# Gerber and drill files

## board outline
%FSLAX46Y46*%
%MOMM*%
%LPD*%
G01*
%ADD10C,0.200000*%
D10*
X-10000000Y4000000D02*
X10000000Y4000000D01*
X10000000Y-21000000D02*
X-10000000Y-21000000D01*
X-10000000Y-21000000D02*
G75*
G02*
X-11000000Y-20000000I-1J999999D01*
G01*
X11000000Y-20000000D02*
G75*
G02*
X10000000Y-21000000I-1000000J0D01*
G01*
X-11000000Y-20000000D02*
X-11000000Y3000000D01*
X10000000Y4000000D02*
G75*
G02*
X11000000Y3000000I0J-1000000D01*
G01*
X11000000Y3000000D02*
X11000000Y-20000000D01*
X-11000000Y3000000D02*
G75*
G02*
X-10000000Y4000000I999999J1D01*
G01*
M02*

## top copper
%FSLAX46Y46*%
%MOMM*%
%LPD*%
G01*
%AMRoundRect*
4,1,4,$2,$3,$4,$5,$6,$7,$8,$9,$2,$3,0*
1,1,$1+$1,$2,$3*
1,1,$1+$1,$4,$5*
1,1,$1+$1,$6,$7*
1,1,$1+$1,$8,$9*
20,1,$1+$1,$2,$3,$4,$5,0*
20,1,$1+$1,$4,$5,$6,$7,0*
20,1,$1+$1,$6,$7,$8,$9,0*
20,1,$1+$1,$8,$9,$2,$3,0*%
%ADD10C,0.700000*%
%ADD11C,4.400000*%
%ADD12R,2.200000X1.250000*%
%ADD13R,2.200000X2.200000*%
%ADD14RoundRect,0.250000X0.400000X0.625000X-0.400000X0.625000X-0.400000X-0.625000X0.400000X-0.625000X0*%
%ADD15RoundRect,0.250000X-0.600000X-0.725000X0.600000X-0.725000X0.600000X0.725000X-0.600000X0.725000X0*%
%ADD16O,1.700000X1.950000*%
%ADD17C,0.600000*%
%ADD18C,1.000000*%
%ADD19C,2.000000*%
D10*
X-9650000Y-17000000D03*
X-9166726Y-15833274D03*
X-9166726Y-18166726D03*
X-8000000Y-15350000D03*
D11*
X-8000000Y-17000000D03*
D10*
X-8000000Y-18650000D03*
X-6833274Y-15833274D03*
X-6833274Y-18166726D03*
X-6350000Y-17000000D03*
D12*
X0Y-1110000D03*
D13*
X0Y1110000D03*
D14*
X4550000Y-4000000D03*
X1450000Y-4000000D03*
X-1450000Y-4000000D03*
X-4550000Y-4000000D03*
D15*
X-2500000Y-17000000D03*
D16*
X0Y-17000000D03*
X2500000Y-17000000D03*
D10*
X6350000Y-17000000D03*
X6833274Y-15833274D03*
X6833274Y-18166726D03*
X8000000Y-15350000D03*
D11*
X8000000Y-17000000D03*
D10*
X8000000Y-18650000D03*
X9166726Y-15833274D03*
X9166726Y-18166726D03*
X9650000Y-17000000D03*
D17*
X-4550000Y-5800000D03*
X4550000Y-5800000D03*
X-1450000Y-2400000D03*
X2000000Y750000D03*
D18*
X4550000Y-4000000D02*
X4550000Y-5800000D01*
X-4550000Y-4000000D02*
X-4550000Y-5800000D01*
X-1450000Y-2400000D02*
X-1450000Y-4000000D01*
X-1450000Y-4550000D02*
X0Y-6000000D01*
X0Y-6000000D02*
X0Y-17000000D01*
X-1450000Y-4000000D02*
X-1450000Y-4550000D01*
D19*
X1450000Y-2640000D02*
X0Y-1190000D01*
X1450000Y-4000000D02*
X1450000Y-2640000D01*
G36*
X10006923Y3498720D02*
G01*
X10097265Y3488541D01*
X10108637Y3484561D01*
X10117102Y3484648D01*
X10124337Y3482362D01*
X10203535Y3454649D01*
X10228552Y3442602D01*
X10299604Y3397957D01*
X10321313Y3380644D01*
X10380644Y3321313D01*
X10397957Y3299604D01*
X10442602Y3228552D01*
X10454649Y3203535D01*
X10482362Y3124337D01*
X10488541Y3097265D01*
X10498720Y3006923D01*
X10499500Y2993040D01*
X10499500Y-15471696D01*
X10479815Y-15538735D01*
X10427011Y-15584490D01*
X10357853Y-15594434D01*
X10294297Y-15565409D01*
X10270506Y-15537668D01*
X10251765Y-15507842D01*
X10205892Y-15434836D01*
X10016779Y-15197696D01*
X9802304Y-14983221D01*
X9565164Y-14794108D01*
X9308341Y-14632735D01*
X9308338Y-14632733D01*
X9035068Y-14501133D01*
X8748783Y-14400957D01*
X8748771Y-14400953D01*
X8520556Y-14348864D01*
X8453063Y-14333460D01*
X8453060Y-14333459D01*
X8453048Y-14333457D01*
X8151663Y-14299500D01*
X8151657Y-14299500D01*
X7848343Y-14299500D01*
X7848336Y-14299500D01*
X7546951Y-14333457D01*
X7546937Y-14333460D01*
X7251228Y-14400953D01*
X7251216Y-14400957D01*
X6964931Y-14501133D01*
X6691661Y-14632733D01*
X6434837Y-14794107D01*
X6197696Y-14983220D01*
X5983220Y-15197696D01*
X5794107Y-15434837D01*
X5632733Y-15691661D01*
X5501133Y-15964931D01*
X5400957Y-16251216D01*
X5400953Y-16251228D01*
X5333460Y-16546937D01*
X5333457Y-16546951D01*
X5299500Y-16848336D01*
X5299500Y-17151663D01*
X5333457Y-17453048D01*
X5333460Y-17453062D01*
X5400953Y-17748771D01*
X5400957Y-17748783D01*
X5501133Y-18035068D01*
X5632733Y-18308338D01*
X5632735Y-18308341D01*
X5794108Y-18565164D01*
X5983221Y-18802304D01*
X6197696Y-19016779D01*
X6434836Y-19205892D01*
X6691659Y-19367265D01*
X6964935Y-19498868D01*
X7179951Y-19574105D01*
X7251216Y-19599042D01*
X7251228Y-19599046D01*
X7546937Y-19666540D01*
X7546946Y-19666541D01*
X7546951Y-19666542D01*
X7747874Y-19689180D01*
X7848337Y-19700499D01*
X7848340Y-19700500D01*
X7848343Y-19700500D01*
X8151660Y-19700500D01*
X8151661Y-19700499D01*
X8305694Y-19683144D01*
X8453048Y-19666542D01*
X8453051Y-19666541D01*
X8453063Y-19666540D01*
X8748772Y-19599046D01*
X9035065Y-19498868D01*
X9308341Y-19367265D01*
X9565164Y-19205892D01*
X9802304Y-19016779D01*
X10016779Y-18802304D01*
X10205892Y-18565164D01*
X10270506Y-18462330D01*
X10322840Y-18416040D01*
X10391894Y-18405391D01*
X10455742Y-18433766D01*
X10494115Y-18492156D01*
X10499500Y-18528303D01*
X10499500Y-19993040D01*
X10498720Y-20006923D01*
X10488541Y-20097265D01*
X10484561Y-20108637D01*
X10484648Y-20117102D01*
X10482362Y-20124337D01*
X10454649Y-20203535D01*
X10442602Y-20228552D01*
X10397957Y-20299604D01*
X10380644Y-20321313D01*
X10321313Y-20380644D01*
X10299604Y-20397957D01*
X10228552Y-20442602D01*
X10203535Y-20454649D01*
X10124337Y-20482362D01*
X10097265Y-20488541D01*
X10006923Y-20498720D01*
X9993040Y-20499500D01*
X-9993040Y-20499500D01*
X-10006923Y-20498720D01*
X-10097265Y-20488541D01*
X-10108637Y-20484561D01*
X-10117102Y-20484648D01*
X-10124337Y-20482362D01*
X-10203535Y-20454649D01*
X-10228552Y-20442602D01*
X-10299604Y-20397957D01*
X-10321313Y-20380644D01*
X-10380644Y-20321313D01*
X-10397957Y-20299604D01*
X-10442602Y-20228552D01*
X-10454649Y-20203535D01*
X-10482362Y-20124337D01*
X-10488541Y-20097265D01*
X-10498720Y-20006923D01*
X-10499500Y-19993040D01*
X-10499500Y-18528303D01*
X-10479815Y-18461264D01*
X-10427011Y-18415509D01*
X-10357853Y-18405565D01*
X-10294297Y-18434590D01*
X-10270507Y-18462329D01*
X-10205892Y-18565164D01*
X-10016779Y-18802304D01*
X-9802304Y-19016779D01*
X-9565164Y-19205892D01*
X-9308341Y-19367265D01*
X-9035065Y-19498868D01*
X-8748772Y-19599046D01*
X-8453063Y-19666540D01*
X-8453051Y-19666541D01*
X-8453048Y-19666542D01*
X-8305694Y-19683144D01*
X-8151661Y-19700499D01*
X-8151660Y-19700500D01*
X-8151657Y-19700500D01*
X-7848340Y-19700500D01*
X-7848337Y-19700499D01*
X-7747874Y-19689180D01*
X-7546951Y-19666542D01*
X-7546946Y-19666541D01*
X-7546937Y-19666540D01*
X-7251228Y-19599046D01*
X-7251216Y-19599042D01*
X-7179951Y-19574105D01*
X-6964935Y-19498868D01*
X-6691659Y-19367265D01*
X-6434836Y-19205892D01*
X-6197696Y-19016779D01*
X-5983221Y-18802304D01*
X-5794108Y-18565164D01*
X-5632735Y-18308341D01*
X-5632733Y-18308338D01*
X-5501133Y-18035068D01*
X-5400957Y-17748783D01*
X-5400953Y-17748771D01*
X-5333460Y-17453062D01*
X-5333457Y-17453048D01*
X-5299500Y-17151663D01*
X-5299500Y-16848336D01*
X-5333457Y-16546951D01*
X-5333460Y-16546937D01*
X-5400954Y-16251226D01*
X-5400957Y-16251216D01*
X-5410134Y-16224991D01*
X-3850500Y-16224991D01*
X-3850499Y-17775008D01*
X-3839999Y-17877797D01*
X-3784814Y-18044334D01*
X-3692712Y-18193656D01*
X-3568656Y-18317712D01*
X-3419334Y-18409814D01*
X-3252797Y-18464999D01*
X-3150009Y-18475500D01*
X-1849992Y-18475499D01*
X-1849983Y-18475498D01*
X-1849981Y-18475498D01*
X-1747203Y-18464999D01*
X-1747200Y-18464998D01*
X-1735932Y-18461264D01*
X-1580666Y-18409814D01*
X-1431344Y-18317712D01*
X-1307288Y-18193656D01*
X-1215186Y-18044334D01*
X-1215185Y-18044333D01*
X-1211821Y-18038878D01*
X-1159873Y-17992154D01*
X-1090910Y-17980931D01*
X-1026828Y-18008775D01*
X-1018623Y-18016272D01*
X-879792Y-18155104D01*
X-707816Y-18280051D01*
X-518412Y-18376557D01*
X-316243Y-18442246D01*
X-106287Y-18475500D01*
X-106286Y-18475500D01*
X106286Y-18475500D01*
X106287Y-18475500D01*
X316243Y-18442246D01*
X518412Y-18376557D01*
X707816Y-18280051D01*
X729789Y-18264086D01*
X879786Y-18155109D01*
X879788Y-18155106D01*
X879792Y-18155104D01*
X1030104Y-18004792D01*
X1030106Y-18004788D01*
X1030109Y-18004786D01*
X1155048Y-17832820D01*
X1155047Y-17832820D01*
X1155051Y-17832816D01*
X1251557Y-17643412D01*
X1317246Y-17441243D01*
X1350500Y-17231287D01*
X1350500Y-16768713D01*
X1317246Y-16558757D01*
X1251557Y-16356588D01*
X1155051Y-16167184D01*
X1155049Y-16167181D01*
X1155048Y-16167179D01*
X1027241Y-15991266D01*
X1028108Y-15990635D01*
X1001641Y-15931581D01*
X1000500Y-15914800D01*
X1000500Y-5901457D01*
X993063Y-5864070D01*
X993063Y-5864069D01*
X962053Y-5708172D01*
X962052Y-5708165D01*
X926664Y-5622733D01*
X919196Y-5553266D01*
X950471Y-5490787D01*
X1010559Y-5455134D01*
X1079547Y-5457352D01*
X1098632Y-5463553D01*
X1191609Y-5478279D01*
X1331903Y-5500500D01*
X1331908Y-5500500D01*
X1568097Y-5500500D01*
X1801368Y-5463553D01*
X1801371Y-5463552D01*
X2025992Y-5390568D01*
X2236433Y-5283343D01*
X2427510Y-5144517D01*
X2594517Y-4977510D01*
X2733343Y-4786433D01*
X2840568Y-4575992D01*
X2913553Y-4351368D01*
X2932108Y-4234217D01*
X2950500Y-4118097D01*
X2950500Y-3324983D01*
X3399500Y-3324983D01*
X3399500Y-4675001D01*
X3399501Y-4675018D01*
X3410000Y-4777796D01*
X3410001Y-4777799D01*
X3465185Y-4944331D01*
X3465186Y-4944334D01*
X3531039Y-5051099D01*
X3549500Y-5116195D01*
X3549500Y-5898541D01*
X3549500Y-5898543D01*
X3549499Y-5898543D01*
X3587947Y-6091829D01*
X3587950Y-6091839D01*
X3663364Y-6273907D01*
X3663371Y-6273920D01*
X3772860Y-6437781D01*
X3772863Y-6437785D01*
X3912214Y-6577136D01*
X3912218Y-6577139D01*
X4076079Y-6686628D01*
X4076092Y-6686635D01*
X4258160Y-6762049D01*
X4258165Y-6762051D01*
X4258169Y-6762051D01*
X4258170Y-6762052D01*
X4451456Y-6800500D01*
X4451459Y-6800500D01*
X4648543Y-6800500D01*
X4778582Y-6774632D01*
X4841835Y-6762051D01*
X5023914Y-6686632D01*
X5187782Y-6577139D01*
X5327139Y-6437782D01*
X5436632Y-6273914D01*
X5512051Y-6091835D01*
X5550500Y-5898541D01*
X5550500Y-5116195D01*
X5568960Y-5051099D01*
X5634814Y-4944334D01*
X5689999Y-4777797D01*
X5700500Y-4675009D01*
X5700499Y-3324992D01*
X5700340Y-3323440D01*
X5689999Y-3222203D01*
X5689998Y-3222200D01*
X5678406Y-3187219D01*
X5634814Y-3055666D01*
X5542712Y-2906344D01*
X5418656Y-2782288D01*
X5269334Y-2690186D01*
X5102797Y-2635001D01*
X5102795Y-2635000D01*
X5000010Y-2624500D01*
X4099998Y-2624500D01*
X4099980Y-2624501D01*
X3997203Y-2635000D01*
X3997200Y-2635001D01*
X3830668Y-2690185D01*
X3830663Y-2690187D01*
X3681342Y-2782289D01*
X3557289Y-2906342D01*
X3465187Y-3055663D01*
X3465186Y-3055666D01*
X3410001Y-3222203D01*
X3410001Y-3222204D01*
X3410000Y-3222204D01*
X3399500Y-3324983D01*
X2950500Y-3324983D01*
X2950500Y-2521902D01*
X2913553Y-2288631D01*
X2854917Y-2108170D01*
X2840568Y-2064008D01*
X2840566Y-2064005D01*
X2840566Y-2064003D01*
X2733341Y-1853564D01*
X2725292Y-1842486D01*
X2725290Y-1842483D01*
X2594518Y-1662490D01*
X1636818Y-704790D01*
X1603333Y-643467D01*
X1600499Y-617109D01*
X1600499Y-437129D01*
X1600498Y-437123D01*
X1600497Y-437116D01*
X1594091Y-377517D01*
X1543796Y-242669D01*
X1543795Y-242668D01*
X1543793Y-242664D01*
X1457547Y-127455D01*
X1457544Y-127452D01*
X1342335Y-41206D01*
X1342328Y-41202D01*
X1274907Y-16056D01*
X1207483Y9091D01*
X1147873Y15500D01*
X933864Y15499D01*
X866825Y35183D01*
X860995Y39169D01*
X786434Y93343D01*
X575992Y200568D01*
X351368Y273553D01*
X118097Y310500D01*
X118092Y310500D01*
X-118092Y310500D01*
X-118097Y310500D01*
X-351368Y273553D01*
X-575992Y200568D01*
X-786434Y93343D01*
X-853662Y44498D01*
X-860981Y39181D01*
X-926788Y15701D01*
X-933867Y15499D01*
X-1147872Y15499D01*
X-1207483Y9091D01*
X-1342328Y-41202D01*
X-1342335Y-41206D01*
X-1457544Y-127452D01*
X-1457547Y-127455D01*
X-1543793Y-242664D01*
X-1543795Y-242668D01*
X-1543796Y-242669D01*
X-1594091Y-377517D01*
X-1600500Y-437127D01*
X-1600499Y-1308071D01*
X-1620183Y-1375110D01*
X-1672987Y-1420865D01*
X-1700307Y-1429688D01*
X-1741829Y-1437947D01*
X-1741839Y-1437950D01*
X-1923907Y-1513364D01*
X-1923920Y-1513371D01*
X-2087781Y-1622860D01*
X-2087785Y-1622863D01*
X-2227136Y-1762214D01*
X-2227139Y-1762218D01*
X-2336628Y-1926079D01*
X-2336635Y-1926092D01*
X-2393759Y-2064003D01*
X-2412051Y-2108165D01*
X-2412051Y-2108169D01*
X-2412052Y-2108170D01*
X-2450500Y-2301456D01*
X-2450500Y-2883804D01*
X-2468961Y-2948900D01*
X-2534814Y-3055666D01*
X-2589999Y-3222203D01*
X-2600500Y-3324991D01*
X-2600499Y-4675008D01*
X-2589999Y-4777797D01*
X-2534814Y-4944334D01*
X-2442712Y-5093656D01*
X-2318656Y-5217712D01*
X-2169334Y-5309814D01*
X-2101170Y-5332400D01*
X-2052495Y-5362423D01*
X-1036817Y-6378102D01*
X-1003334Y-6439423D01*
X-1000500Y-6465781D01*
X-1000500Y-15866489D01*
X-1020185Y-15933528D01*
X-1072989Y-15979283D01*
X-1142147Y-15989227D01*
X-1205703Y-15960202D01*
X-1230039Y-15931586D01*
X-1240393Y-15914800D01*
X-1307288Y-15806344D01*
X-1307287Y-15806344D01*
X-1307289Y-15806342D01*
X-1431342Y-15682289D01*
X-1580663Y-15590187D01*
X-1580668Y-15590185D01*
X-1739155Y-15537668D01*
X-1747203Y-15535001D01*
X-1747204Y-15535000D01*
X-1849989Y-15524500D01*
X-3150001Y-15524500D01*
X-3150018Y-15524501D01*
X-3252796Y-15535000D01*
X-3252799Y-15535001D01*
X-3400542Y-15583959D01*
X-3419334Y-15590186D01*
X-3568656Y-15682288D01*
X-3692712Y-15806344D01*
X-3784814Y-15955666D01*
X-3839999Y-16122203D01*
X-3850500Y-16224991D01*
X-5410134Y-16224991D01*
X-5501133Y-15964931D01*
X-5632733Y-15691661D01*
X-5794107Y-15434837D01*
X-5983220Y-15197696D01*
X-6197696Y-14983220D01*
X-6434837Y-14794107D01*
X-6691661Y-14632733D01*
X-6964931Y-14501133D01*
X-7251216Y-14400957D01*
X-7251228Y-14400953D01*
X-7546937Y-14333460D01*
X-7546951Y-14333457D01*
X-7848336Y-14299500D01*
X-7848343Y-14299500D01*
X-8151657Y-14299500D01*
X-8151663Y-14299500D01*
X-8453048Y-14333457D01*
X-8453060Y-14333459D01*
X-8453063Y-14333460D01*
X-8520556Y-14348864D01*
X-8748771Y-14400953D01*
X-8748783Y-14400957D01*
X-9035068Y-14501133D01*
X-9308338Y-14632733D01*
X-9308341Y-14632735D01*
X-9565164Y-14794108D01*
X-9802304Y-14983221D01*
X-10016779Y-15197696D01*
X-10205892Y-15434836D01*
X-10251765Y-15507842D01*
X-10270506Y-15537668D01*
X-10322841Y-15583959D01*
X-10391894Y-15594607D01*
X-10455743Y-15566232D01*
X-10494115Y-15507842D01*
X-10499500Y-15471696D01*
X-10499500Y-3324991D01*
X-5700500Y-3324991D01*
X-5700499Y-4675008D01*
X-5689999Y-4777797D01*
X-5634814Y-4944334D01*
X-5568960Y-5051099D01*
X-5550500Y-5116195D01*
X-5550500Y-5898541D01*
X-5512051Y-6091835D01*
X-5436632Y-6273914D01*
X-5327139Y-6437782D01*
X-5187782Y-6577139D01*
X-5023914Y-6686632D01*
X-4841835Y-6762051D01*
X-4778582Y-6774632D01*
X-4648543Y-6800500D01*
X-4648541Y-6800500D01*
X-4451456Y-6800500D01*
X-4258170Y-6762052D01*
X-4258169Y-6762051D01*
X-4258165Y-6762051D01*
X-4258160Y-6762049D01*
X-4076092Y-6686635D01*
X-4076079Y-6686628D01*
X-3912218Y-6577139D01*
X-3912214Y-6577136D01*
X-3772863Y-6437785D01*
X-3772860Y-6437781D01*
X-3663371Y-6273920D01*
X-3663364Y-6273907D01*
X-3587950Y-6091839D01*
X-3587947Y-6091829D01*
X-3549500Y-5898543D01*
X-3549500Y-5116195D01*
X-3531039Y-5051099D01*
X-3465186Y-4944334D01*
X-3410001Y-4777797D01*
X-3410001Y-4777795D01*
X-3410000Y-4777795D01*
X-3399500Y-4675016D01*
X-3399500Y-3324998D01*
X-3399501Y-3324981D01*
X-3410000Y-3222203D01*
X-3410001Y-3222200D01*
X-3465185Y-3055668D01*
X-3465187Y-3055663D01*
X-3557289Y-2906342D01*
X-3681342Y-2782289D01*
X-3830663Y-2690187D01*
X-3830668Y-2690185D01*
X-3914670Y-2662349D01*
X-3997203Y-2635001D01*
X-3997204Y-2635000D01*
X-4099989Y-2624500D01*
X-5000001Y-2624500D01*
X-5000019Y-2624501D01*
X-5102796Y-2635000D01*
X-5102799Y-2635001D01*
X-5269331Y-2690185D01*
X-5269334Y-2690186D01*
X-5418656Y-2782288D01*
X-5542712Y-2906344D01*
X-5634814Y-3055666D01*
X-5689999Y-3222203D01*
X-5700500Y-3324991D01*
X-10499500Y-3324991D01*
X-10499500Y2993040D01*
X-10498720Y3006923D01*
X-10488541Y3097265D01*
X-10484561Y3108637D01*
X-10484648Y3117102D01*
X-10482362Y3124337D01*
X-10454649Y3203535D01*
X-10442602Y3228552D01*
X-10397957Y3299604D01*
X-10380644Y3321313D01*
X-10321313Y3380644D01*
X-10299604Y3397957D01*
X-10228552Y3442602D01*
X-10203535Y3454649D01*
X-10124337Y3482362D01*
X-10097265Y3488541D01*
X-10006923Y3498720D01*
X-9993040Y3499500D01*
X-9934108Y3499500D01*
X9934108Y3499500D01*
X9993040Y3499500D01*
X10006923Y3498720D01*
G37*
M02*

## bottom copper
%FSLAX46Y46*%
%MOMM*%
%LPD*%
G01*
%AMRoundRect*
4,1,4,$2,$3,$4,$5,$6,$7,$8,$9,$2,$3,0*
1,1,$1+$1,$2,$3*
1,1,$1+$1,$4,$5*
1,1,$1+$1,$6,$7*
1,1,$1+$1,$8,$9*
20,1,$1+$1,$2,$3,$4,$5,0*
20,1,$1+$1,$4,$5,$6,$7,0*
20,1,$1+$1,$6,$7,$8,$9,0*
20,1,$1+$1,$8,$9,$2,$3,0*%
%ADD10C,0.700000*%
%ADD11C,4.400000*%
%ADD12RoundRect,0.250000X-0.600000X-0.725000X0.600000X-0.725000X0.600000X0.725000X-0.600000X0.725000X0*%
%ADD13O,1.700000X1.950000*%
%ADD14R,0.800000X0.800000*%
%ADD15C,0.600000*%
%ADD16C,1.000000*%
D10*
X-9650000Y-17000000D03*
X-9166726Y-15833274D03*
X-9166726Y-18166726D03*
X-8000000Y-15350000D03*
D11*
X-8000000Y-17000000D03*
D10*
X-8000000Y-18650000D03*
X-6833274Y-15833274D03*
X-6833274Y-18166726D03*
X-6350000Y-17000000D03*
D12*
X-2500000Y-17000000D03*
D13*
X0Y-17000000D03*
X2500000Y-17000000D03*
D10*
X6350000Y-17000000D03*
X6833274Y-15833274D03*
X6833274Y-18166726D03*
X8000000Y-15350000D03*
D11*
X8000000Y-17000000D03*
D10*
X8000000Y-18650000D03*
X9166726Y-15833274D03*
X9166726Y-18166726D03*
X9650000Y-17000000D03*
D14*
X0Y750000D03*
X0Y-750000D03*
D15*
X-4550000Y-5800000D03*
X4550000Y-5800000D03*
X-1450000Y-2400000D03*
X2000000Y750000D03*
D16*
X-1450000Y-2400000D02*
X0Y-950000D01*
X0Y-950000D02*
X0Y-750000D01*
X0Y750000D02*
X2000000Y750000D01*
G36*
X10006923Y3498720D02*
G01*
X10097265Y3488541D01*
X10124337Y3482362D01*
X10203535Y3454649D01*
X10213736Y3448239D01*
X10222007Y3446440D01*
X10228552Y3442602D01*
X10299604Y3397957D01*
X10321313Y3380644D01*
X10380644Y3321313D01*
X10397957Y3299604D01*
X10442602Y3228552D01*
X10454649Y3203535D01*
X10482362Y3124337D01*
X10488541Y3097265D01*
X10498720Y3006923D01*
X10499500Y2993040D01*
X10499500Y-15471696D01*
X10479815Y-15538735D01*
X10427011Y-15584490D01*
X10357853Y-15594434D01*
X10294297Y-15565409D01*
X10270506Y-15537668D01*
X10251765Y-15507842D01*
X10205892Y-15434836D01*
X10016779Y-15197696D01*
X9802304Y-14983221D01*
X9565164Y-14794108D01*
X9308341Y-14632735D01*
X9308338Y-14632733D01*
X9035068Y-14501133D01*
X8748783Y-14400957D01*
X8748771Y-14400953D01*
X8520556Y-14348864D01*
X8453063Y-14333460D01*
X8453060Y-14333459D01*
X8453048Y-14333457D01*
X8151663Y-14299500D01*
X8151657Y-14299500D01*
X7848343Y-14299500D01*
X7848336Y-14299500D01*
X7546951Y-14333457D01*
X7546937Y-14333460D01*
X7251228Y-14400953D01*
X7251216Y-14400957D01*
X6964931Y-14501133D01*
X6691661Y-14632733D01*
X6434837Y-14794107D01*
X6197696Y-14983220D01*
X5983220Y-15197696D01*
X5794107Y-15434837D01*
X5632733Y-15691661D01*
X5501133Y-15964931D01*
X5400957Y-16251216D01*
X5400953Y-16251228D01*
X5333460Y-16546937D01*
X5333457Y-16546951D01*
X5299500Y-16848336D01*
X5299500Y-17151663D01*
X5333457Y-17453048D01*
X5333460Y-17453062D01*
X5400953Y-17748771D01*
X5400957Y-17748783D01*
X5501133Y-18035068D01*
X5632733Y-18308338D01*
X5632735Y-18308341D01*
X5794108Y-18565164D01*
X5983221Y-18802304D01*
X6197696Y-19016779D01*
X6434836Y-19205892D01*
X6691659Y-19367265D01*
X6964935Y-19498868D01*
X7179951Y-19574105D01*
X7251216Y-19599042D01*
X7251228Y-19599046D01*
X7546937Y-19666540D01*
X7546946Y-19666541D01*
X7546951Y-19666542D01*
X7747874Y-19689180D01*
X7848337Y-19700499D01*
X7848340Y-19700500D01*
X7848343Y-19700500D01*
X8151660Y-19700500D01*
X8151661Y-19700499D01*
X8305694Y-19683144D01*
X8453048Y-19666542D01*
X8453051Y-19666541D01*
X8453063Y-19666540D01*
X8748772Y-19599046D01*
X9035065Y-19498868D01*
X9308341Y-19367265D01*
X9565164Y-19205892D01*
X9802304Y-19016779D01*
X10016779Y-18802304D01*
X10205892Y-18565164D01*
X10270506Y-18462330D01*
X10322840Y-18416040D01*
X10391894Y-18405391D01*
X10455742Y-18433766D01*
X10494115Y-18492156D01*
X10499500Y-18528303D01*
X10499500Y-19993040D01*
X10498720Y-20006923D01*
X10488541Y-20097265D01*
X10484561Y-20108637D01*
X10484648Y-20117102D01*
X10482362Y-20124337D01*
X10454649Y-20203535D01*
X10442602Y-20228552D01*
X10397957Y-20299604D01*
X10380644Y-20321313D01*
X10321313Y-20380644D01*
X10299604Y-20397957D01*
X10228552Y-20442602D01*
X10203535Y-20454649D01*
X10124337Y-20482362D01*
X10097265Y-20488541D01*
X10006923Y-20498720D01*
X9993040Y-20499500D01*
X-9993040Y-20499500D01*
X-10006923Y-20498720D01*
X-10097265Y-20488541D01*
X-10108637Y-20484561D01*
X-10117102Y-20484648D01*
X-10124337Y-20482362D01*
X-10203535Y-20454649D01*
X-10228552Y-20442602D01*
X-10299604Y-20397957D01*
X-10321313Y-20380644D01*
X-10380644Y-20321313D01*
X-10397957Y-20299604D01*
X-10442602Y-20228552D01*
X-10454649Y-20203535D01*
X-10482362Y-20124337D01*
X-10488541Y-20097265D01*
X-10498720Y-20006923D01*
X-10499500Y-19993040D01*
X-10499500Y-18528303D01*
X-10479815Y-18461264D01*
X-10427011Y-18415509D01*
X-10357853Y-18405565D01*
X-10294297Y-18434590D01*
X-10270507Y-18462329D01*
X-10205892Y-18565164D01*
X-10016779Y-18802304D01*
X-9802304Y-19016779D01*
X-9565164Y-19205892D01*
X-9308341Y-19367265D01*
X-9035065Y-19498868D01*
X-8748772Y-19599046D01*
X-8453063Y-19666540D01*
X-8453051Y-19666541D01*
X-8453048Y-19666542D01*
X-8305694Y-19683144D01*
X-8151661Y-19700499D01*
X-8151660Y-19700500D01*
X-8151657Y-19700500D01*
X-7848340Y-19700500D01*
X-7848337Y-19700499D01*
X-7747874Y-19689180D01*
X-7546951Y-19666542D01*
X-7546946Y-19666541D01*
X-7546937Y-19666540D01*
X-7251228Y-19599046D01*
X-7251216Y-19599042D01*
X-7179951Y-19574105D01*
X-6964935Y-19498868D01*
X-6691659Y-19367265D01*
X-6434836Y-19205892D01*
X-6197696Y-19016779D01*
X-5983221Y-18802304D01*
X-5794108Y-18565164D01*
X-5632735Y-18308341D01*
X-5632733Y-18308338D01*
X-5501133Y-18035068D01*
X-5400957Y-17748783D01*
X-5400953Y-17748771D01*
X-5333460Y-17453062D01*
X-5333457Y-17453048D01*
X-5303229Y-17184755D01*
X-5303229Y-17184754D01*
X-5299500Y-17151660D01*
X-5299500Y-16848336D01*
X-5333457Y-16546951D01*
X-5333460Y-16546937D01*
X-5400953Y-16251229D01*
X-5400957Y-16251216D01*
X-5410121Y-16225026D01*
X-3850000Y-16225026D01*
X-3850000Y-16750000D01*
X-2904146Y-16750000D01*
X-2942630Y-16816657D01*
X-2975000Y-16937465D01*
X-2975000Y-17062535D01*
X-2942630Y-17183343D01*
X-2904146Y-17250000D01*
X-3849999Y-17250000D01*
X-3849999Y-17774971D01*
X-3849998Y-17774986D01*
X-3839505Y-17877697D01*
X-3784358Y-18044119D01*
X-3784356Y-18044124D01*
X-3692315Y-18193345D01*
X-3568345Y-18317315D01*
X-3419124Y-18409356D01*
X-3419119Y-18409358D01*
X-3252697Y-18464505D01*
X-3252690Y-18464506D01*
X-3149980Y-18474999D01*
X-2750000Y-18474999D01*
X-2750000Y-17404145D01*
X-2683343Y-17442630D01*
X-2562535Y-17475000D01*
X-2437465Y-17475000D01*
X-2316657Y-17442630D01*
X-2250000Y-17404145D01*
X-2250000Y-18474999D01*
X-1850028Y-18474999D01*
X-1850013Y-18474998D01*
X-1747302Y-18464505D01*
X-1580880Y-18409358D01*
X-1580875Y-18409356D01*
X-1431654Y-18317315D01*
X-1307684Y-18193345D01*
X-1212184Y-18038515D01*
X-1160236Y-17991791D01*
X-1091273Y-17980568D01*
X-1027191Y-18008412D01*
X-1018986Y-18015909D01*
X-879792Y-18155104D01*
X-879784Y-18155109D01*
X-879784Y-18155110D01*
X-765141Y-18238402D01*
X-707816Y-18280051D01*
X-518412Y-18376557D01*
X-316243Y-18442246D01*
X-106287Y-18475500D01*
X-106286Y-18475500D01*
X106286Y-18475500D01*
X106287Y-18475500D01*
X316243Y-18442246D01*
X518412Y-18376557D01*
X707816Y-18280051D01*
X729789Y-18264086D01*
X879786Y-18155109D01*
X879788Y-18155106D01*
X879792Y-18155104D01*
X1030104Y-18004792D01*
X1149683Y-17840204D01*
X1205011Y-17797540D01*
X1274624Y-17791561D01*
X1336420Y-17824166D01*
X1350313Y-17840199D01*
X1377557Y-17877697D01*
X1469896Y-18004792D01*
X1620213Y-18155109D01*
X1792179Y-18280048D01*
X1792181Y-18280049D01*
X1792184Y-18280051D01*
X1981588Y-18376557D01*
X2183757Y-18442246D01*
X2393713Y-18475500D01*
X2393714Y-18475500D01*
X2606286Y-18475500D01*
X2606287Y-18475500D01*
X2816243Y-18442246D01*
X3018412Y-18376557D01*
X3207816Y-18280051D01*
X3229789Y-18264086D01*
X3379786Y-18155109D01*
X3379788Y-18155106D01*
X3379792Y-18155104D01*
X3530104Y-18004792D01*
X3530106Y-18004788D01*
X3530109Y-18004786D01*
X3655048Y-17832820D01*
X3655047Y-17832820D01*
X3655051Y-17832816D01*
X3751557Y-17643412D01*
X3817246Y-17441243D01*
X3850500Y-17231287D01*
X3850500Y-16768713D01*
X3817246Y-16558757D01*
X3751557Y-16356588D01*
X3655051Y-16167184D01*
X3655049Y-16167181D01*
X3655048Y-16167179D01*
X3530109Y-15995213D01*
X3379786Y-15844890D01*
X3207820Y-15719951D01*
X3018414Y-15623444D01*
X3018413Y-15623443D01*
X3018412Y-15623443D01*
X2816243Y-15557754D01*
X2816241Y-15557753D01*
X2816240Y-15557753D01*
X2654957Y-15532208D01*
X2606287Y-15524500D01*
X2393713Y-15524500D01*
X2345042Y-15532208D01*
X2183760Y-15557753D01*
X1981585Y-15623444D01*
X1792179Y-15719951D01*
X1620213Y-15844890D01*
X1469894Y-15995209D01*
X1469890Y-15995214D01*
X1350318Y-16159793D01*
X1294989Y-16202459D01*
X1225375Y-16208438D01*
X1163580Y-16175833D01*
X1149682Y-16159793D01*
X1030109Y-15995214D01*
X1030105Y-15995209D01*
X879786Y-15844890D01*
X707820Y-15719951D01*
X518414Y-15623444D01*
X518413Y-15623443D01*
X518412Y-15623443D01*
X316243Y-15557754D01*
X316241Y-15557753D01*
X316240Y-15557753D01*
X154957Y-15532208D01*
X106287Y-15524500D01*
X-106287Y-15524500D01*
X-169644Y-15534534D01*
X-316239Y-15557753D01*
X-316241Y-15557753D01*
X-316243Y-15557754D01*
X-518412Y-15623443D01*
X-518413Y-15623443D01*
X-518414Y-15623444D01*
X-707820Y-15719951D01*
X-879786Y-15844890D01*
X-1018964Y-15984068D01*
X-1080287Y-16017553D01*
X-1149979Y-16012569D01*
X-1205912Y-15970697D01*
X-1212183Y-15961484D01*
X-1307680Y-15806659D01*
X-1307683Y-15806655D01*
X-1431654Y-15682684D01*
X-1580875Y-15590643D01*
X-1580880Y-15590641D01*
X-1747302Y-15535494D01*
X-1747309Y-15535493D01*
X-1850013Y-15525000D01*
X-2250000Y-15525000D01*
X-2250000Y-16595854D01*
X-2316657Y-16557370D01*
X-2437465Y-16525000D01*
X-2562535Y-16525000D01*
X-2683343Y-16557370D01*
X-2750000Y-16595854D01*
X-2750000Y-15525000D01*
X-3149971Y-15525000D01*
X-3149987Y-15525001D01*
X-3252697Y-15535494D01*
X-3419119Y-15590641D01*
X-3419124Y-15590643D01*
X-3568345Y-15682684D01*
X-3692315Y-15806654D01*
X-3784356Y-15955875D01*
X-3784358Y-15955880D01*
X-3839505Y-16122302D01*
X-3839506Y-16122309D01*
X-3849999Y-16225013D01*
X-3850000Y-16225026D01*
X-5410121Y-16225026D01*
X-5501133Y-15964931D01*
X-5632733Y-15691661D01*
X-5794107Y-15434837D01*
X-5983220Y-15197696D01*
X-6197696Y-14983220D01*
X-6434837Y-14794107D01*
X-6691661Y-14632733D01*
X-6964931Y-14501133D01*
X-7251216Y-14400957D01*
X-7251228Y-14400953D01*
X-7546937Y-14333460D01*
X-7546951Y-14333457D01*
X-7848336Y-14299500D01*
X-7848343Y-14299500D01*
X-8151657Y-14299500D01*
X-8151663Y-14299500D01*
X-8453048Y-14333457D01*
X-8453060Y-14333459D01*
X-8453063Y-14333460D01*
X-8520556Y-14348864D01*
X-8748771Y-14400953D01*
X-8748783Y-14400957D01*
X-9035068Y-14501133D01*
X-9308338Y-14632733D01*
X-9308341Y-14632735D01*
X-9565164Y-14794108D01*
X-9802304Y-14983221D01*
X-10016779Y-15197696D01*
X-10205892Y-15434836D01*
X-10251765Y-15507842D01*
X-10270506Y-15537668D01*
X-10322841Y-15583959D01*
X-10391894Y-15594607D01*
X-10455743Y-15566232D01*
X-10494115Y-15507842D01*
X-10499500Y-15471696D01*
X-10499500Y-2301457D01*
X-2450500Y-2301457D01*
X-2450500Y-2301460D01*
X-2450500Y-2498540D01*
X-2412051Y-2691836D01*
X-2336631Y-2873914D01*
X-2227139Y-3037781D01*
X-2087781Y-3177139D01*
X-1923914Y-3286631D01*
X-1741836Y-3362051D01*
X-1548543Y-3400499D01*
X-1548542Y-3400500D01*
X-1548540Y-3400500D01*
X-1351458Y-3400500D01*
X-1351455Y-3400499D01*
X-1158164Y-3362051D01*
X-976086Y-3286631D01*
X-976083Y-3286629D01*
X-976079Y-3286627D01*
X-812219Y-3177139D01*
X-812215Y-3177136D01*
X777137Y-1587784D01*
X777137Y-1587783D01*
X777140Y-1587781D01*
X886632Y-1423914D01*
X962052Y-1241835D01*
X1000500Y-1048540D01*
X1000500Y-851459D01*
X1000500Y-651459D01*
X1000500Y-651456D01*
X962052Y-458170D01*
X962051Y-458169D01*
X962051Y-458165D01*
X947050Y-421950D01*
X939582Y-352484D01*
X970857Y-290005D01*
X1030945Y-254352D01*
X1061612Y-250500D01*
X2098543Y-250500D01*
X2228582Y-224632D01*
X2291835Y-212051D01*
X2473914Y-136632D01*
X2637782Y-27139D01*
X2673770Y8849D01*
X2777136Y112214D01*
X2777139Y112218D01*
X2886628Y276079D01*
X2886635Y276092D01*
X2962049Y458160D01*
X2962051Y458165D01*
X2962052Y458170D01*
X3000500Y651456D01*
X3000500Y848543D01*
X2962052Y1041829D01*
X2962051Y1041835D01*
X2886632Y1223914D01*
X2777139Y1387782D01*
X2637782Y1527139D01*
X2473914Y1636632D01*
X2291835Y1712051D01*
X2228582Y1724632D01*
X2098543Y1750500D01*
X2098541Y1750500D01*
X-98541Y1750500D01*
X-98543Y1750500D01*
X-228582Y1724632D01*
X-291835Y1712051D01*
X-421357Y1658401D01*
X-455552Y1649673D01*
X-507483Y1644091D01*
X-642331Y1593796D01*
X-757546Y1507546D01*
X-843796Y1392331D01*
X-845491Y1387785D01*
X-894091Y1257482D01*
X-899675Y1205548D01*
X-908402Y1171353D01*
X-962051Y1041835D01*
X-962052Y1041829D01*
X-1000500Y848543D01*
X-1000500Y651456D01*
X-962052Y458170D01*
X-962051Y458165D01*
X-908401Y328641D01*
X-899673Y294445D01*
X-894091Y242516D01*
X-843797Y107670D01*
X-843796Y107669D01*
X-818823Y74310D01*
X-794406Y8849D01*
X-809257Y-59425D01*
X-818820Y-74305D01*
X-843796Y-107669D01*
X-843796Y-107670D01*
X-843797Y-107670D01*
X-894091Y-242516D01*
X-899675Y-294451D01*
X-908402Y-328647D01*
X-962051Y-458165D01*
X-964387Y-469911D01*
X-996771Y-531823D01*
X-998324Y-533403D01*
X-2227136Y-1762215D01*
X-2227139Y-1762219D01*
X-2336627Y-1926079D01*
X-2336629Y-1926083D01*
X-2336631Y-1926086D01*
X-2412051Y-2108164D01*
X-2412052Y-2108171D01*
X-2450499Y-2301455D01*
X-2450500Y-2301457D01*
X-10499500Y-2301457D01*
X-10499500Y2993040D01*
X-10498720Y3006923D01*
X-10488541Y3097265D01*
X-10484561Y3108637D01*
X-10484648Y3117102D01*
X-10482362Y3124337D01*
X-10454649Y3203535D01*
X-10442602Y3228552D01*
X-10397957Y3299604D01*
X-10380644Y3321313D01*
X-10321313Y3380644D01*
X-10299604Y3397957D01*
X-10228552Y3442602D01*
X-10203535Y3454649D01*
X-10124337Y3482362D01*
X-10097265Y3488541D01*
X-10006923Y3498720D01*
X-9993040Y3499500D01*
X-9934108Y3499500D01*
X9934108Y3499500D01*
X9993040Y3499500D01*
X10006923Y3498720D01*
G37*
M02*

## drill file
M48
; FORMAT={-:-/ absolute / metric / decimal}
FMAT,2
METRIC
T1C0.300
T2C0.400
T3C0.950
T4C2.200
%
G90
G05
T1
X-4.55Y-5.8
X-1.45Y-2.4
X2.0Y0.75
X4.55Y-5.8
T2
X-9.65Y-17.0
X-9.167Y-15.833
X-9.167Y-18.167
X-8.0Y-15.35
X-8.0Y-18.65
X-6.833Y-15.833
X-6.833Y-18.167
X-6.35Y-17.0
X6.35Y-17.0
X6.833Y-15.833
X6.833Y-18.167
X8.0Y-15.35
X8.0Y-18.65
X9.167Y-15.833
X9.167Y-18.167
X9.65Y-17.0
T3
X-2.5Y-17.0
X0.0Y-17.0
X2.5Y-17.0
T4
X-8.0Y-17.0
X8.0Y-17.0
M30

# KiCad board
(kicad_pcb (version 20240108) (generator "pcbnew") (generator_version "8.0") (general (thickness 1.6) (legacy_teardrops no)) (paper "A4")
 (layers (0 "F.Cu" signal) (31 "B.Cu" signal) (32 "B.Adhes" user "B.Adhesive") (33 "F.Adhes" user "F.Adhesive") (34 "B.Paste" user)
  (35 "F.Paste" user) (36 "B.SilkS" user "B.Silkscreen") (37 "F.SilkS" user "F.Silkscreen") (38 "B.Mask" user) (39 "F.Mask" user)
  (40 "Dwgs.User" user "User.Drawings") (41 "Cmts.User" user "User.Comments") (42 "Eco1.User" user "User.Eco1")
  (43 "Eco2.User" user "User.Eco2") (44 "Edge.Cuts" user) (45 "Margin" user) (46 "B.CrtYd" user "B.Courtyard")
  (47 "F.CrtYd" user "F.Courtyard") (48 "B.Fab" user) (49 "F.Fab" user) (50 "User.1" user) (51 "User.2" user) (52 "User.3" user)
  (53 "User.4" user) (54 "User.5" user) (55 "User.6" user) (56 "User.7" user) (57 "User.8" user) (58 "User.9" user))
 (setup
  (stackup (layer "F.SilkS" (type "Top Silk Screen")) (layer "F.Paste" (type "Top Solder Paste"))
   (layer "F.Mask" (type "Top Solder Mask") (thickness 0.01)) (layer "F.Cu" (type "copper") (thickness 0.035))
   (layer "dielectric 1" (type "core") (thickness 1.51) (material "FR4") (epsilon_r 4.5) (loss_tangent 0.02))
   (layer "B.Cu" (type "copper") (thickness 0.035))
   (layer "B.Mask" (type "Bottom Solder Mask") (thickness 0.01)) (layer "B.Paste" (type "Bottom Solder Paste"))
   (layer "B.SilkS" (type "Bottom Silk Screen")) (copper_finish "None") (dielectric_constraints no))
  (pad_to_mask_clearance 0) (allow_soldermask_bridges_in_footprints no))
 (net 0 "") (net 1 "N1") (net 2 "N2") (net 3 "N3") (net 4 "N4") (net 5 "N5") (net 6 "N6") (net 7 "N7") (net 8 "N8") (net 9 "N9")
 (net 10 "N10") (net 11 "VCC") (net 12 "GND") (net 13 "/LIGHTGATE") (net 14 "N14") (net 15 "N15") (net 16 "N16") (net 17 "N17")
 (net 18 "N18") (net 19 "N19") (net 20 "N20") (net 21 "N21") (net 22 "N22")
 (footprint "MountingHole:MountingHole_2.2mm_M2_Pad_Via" (layer "F.Cu") (at -8 17)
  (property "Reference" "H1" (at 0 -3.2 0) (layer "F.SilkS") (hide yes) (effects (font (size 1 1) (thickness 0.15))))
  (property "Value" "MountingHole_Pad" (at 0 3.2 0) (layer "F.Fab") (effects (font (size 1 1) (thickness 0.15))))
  (pad "1" thru_hole circle (at -1.65 0) (size 0.7 0.7) (drill 0.4) (layers "*.Cu" "*.Mask") (remove_unused_layers no) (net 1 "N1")
   (zone_connect 2))
  (pad "1" thru_hole circle (at -1.166726 -1.166726) (size 0.7 0.7) (drill 0.4) (layers "*.Cu" "*.Mask") (remove_unused_layers no)
   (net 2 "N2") (zone_connect 2))
  (pad "1" thru_hole circle (at -1.166726 1.166726) (size 0.7 0.7) (drill 0.4) (layers "*.Cu" "*.Mask") (remove_unused_layers no)
   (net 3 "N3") (zone_connect 2))
  (pad "1" thru_hole circle (at 0 -1.65) (size 0.7 0.7) (drill 0.4) (layers "*.Cu" "*.Mask") (remove_unused_layers no) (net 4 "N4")
   (zone_connect 2))
  (pad "1" thru_hole circle (at 0 0) (size 4.4 4.4) (drill 2.2) (layers "*.Cu" "*.Mask") (remove_unused_layers no) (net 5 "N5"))
  (pad "1" thru_hole circle (at 0 1.65) (size 0.7 0.7) (drill 0.4) (layers "*.Cu" "*.Mask") (remove_unused_layers no) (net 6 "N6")
   (zone_connect 2))
  (pad "1" thru_hole circle (at 1.166726 -1.166726) (size 0.7 0.7) (drill 0.4) (layers "*.Cu" "*.Mask") (remove_unused_layers no)
   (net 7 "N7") (zone_connect 2))
  (pad "1" thru_hole circle (at 1.166726 1.166726) (size 0.7 0.7) (drill 0.4) (layers "*.Cu" "*.Mask") (remove_unused_layers no)
   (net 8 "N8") (zone_connect 2))
  (pad "1" thru_hole circle (at 1.65 0) (size 0.7 0.7) (drill 0.4) (layers "*.Cu" "*.Mask") (remove_unused_layers no) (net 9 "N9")
   (zone_connect 2)))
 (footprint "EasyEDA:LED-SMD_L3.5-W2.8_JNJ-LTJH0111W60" (layer "F.Cu") (at 0 0 90)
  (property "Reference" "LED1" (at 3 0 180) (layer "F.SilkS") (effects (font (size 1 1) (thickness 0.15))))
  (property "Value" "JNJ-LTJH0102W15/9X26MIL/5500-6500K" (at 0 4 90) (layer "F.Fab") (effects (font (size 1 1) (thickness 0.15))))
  (pad "1" smd rect (at -1.11 0 270) (size 1.25 2.2) (layers "F.Cu" "F.Paste" "F.Mask") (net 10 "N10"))
  (pad "2" smd rect (at 1.11 0 270) (size 2.2 2.2) (layers "F.Cu" "F.Paste" "F.Mask") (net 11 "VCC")))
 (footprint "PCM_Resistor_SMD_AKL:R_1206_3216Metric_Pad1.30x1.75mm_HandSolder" (layer "F.Cu") (at 3 4 180)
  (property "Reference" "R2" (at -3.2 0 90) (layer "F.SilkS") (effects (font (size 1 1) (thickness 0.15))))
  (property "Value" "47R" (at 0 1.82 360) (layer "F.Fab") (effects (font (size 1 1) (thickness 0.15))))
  (pad "1" smd roundrect (at -1.55 0 180) (size 1.3 1.75) (layers "F.Cu" "F.Paste" "F.Mask") (roundrect_rratio 0.192308) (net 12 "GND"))
  (pad "2" smd roundrect (at 1.55 0 180) (size 1.3 1.75) (layers "F.Cu" "F.Paste" "F.Mask") (roundrect_rratio 0.192308) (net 10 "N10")))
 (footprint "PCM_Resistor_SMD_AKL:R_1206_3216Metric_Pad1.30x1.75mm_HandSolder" (layer "F.Cu") (at -3 4 180)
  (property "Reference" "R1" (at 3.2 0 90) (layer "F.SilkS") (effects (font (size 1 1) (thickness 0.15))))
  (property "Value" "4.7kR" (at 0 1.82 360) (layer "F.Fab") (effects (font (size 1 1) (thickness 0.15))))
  (pad "1" smd roundrect (at -1.55 0 180) (size 1.3 1.75) (layers "F.Cu" "F.Paste" "F.Mask") (roundrect_rratio 0.192308)
   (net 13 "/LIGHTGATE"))
  (pad "2" smd roundrect (at 1.55 0 180) (size 1.3 1.75) (layers "F.Cu" "F.Paste" "F.Mask") (roundrect_rratio 0.192308) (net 12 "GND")))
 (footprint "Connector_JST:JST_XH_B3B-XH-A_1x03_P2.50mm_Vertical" (layer "F.Cu") (at -2.5 17)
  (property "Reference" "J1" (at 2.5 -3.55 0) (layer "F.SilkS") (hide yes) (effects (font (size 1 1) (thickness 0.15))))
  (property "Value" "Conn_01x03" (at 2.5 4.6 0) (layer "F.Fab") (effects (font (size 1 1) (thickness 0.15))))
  (pad "1" thru_hole roundrect (at 0 0) (size 1.7 1.95) (drill 0.95) (layers "*.Cu" "*.Mask") (remove_unused_layers no)
   (roundrect_rratio 0.147059) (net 12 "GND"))
  (pad "2" thru_hole oval (at 2.5 0) (size 1.7 1.95) (drill 0.95) (layers "*.Cu" "*.Mask") (remove_unused_layers no) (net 13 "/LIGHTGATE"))
  (pad "3" thru_hole oval (at 5 0) (size 1.7 1.95) (drill 0.95) (layers "*.Cu" "*.Mask") (remove_unused_layers no) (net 11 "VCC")))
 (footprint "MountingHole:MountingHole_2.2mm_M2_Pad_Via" (layer "F.Cu") (at 8 17)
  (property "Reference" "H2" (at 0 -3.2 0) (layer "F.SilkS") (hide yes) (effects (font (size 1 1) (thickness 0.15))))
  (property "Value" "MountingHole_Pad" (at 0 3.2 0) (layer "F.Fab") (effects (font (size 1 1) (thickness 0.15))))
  (pad "1" thru_hole circle (at -1.65 0) (size 0.7 0.7) (drill 0.4) (layers "*.Cu" "*.Mask") (remove_unused_layers no) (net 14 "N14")
   (zone_connect 2))
  (pad "1" thru_hole circle (at -1.166726 -1.166726) (size 0.7 0.7) (drill 0.4) (layers "*.Cu" "*.Mask") (remove_unused_layers no)
   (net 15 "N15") (zone_connect 2))
  (pad "1" thru_hole circle (at -1.166726 1.166726) (size 0.7 0.7) (drill 0.4) (layers "*.Cu" "*.Mask") (remove_unused_layers no)
   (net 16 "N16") (zone_connect 2))
  (pad "1" thru_hole circle (at 0 -1.65) (size 0.7 0.7) (drill 0.4) (layers "*.Cu" "*.Mask") (remove_unused_layers no) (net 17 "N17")
   (zone_connect 2))
  (pad "1" thru_hole circle (at 0 0) (size 4.4 4.4) (drill 2.2) (layers "*.Cu" "*.Mask") (remove_unused_layers no) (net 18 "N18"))
  (pad "1" thru_hole circle (at 0 1.65) (size 0.7 0.7) (drill 0.4) (layers "*.Cu" "*.Mask") (remove_unused_layers no) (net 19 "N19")
   (zone_connect 2))
  (pad "1" thru_hole circle (at 1.166726 -1.166726) (size 0.7 0.7) (drill 0.4) (layers "*.Cu" "*.Mask") (remove_unused_layers no)
   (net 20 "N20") (zone_connect 2))
  (pad "1" thru_hole circle (at 1.166726 1.166726) (size 0.7 0.7) (drill 0.4) (layers "*.Cu" "*.Mask") (remove_unused_layers no)
   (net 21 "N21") (zone_connect 2))
  (pad "1" thru_hole circle (at 1.65 0) (size 0.7 0.7) (drill 0.4) (layers "*.Cu" "*.Mask") (remove_unused_layers no) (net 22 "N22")
   (zone_connect 2)))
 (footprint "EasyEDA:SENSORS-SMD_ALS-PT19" (layer "B.Cu") (at 0 0 -90)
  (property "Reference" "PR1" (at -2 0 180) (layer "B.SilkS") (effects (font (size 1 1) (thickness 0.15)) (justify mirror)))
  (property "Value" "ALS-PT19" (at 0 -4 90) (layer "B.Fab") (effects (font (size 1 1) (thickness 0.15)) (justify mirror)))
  (pad "1" smd rect (at -0.75 0 90) (size 0.8 0.8) (layers "B.Cu" "B.Paste" "B.Mask") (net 11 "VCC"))
  (pad "2" smd rect (at 0.75 0 90) (size 0.8 0.8) (layers "B.Cu" "B.Paste" "B.Mask") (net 13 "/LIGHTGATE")))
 (gr_line (start -10 -4) (end 10 -4) (stroke (width 0.2) (type default)) (layer "Edge.Cuts"))
 (gr_line (start 10 21) (end -10 21) (stroke (width 0.2) (type default)) (layer "Edge.Cuts"))
 (gr_arc (start -10 21) (mid -10.707107 20.707107) (end -11 20) (stroke (width 0.2) (type default)) (layer "Edge.Cuts"))
 (gr_arc (start 11 20) (mid 10.707107 20.707107) (end 10 21) (stroke (width 0.2) (type default)) (layer "Edge.Cuts"))
 (gr_line (start -11 20) (end -11 -3) (stroke (width 0.2) (type default)) (layer "Edge.Cuts"))
 (gr_arc (start 10 -4) (mid 10.707107 -3.707107) (end 11 -3) (stroke (width 0.2) (type default)) (layer "Edge.Cuts"))
 (gr_line (start 11 -3) (end 11 20) (stroke (width 0.2) (type default)) (layer "Edge.Cuts"))
 (gr_arc (start -11 -3) (mid -10.707107 -3.707107) (end -10 -4) (stroke (width 0.2) (type default)) (layer "Edge.Cuts"))
 (segment (start 4.55 4) (end 4.55 5.8) (width 1) (layer "F.Cu") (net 12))
 (segment (start -4.55 4) (end -4.55 5.8) (width 1) (layer "F.Cu") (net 12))
 (via (at -4.55 5.8) (size 0.6) (drill 0.3) (layers "F.Cu" "B.Cu") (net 12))
 (via (at 4.55 5.8) (size 0.6) (drill 0.3) (layers "F.Cu" "B.Cu") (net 12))
 (segment (start -1.45 2.4) (end -1.45 4) (width 1) (layer "F.Cu") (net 13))
 (segment (start -1.45 4.55) (end 0 6) (width 1) (layer "F.Cu") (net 13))
 (segment (start 0 6) (end 0 17) (width 1) (layer "F.Cu") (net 13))
 (segment (start -1.45 4) (end -1.45 4.55) (width 1) (layer "F.Cu") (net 13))
 (via (at -1.45 2.4) (size 0.6) (drill 0.3) (layers "F.Cu" "B.Cu") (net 13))
 (segment (start -1.45 2.4) (end 0 0.95) (width 1) (layer "B.Cu") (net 13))
 (segment (start 0 0.95) (end 0 0.75) (width 1) (layer "B.Cu") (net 13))
 (via (at 2 -0.75) (size 0.6) (drill 0.3) (layers "F.Cu" "B.Cu") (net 11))
 (segment (start 0 -0.75) (end 2 -0.75) (width 1) (layer "B.Cu") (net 11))
 (segment (start 1.45 2.64) (end 0 1.19) (width 2) (layer "F.Cu") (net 10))
 (segment (start 1.45 4) (end 1.45 2.64) (width 2) (layer "F.Cu") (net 10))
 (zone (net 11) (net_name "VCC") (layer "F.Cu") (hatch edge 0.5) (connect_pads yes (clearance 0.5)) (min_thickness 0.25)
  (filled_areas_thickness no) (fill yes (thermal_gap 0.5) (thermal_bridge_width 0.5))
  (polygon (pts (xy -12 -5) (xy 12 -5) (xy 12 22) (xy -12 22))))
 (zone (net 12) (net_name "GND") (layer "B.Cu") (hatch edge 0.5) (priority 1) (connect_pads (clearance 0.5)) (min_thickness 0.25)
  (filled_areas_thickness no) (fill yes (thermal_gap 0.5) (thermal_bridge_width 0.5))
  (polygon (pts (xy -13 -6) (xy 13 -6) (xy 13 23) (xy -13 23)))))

